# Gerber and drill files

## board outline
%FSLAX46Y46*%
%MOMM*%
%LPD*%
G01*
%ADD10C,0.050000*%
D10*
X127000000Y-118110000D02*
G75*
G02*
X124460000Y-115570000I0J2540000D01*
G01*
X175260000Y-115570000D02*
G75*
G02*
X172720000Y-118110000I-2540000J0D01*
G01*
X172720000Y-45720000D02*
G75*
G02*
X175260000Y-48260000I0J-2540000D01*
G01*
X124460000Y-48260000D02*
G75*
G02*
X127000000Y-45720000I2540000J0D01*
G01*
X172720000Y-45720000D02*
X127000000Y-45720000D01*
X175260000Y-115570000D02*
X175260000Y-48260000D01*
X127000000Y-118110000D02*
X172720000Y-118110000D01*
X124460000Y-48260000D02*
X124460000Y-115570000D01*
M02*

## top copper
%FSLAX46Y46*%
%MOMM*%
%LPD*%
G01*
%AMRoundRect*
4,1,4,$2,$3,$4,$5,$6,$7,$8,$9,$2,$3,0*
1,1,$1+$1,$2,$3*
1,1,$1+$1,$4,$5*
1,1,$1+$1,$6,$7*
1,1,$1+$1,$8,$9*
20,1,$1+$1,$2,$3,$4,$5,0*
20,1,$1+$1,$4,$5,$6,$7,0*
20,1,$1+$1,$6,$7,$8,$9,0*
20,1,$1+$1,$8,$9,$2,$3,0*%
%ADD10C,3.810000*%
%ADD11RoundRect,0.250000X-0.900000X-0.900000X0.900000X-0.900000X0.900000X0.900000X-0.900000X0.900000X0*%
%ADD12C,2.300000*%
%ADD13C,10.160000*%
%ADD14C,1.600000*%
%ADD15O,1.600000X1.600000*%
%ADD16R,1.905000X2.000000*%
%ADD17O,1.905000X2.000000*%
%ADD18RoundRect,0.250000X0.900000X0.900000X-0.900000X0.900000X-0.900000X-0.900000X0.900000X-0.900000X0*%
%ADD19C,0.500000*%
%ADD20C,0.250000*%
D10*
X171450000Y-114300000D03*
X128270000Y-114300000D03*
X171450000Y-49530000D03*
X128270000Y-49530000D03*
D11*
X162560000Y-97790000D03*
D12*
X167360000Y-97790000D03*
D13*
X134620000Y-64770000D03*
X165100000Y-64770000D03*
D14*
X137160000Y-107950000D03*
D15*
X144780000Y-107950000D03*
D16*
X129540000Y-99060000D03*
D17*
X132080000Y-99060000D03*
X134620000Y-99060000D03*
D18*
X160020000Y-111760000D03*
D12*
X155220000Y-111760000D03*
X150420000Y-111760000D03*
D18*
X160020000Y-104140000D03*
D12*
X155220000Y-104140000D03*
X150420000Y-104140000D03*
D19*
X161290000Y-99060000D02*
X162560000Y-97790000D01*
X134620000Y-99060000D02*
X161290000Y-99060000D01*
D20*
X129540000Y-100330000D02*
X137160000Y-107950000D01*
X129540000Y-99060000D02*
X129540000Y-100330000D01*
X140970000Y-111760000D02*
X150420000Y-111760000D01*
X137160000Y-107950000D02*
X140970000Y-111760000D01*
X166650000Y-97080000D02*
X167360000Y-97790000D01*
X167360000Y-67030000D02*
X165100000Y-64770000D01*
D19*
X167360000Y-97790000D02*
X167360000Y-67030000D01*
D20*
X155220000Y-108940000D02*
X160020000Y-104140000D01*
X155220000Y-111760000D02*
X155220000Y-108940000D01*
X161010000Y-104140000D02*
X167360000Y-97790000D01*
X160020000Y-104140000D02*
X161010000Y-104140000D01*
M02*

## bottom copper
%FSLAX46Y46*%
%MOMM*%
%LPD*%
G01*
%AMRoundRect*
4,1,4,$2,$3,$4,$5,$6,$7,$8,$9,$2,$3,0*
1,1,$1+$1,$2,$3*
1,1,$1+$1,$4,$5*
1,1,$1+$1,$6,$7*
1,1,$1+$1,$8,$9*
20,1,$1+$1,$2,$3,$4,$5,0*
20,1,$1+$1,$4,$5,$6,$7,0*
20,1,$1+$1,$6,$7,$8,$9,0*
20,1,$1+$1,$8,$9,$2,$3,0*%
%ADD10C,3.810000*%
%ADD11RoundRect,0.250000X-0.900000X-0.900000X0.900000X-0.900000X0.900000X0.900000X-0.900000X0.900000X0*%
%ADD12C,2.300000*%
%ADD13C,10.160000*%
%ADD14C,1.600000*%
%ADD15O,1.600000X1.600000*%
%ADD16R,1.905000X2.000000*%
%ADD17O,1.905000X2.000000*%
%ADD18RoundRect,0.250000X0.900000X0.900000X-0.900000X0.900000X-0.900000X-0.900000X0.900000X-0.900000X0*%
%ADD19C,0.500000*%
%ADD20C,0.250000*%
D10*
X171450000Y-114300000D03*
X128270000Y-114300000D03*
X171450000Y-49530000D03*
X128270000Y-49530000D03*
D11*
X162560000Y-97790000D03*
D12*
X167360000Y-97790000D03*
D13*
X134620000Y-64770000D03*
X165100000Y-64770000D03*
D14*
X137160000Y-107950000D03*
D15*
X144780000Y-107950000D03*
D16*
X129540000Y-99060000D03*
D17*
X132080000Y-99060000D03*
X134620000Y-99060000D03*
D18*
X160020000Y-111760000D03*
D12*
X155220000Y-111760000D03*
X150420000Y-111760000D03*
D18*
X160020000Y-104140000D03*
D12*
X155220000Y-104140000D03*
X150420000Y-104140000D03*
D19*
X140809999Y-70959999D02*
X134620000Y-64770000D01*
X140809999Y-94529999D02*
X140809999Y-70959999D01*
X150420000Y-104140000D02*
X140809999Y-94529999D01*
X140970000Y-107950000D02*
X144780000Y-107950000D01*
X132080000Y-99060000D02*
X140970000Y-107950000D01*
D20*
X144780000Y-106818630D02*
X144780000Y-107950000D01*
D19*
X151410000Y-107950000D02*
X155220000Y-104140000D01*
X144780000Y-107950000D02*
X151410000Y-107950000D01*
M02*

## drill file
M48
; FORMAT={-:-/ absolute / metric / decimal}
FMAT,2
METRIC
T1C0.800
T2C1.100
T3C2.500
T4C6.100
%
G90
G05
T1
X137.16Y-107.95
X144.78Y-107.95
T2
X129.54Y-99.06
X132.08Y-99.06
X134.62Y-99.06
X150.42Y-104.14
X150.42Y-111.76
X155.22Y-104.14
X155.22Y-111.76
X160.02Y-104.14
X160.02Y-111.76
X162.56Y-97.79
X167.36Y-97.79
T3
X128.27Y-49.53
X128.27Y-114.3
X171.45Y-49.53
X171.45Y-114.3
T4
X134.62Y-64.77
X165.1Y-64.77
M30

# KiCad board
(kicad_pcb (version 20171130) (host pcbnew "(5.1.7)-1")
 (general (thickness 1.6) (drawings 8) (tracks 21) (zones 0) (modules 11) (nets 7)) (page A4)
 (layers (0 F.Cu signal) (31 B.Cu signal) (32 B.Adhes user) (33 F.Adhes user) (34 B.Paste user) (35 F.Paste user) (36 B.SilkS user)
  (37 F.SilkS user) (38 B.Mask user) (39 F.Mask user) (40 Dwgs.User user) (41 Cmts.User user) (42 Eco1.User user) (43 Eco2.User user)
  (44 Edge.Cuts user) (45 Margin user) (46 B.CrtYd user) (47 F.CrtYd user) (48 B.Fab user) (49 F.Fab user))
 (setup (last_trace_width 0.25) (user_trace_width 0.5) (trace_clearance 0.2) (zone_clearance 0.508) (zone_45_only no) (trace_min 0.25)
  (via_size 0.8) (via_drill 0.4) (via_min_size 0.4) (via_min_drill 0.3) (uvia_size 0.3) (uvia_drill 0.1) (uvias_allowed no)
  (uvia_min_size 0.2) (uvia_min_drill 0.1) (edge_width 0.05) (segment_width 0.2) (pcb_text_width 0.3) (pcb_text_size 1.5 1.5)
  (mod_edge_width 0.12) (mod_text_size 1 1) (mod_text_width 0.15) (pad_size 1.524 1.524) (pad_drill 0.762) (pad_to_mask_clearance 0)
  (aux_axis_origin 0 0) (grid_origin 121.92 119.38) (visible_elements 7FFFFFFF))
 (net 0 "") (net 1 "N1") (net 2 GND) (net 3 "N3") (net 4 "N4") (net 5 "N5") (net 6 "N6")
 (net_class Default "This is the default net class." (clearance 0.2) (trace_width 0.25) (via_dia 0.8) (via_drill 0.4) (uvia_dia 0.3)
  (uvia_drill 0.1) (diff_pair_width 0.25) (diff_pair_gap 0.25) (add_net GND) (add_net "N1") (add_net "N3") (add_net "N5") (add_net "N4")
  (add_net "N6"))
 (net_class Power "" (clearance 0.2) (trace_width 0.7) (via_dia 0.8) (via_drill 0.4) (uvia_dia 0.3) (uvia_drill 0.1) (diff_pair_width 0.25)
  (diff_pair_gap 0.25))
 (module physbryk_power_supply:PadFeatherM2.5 (layer F.Cu) (at 171.45 114.3)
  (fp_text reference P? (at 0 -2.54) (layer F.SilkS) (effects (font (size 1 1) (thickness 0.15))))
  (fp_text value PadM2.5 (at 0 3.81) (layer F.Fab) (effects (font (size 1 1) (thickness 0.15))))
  (pad ? thru_hole circle (at 0 0) (size 3.81 3.81) (drill 2.5) (layers *.Cu *.Mask) (solder_mask_margin 0.0508)))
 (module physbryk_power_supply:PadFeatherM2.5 (layer F.Cu) (at 128.27 114.3)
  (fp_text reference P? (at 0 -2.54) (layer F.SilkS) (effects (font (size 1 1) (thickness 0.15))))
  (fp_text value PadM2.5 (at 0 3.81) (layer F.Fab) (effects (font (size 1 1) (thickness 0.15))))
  (pad ? thru_hole circle (at 0 0) (size 3.81 3.81) (drill 2.5) (layers *.Cu *.Mask) (solder_mask_margin 0.0508)))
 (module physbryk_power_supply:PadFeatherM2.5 (layer F.Cu) (at 171.45 49.53)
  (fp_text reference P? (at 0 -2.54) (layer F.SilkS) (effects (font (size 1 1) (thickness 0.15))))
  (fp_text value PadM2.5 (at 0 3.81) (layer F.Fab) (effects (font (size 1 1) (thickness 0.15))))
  (pad ? thru_hole circle (at 0 0) (size 3.81 3.81) (drill 2.5) (layers *.Cu *.Mask) (solder_mask_margin 0.0508)))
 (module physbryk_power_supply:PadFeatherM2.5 (layer F.Cu) (at 128.27 49.53)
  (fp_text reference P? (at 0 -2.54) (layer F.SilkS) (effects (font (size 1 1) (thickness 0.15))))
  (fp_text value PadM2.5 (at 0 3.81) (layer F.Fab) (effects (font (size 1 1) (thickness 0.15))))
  (pad ? thru_hole circle (at 0 0) (size 3.81 3.81) (drill 2.5) (layers *.Cu *.Mask) (solder_mask_margin 0.0508)))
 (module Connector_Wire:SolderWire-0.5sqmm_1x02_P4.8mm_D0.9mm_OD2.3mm (layer F.Cu) (at 162.56 97.79)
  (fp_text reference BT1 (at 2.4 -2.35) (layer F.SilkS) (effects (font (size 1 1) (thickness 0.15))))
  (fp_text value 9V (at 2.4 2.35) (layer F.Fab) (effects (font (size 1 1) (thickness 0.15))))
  (pad 1 thru_hole roundrect (at 0 0) (size 2.3 2.3) (drill 1.1) (layers *.Cu *.Mask) (roundrect_rratio 0.108695652173913) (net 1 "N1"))
  (pad 2 thru_hole circle (at 4.8 0) (size 2.3 2.3) (drill 1.1) (layers *.Cu *.Mask) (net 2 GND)))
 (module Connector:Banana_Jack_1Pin (layer F.Cu) (at 134.62 64.77)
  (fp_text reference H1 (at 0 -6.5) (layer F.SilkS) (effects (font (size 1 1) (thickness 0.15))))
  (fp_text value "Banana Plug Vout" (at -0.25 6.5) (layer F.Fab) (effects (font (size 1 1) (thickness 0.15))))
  (pad 1 thru_hole circle (at 0 0) (size 10.16 10.16) (drill 6.1) (layers *.Cu *.Mask) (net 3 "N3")))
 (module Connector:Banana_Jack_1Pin (layer F.Cu) (at 165.1 64.77)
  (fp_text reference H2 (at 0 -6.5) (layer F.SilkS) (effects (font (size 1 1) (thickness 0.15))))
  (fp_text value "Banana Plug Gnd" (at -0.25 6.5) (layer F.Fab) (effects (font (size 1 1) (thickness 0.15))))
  (pad 1 thru_hole circle (at 0 0) (size 10.16 10.16) (drill 6.1) (layers *.Cu *.Mask) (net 2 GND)))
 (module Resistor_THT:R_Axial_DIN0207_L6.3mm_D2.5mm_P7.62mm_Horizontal (layer F.Cu) (at 137.16 107.95)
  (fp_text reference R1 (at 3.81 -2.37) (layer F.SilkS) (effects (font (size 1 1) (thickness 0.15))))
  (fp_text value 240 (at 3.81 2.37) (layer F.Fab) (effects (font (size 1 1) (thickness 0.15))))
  (pad 1 thru_hole circle (at 0 0) (size 1.6 1.6) (drill 0.8) (layers *.Cu *.Mask) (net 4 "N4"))
  (pad 2 thru_hole oval (at 7.62 0) (size 1.6 1.6) (drill 0.8) (layers *.Cu *.Mask) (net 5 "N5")))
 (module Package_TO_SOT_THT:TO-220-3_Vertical (layer F.Cu) (at 129.54 99.06)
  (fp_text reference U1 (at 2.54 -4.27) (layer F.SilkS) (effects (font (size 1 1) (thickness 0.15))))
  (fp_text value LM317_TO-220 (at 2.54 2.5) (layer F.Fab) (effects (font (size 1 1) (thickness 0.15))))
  (pad 1 thru_hole rect (at 0 0) (size 1.905 2) (drill 1.1) (layers *.Cu *.Mask) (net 4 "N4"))
  (pad 2 thru_hole oval (at 2.54 0) (size 1.905 2) (drill 1.1) (layers *.Cu *.Mask) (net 5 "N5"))
  (pad 3 thru_hole oval (at 5.08 0) (size 1.905 2) (drill 1.1) (layers *.Cu *.Mask) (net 1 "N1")))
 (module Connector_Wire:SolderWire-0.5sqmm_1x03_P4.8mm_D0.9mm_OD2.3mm (layer F.Cu) (at 160.02 111.76 180)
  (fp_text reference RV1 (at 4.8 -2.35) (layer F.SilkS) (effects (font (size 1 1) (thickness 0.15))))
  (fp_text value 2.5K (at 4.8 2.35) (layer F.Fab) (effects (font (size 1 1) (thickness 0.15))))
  (pad 1 thru_hole roundrect (at 0 0 180) (size 2.3 2.3) (drill 1.1) (layers *.Cu *.Mask) (roundrect_rratio 0.108695652173913) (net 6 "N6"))
  (pad 2 thru_hole circle (at 4.8 0 180) (size 2.3 2.3) (drill 1.1) (layers *.Cu *.Mask) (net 2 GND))
  (pad 3 thru_hole circle (at 9.6 0 180) (size 2.3 2.3) (drill 1.1) (layers *.Cu *.Mask) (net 4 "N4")))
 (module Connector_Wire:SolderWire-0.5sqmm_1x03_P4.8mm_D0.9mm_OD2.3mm (layer F.Cu) (at 160.02 104.14 180)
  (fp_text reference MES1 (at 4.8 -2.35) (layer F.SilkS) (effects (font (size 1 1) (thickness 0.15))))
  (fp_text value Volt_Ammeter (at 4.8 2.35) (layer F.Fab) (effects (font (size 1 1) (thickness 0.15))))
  (pad 1 thru_hole roundrect (at 0 0 180) (size 2.3 2.3) (drill 1.1) (layers *.Cu *.Mask) (roundrect_rratio 0.108695652173913) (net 2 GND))
  (pad 2 thru_hole circle (at 4.8 0 180) (size 2.3 2.3) (drill 1.1) (layers *.Cu *.Mask) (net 5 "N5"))
  (pad 3 thru_hole circle (at 9.6 0 180) (size 2.3 2.3) (drill 1.1) (layers *.Cu *.Mask) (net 3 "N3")))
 (gr_arc (start 127 115.57) (end 124.46 115.57) (angle -90) (layer Edge.Cuts) (width 0.05))
 (gr_arc (start 172.72 115.57) (end 172.72 118.11) (angle -90) (layer Edge.Cuts) (width 0.05))
 (gr_arc (start 172.72 48.26) (end 175.26 48.26) (angle -90) (layer Edge.Cuts) (width 0.05))
 (gr_arc (start 127 48.26) (end 127 45.72) (angle -90) (layer Edge.Cuts) (width 0.05))
 (gr_line (start 172.72 45.72) (end 127 45.72) (layer Edge.Cuts) (width 0.05))
 (gr_line (start 175.26 115.57) (end 175.26 48.26) (layer Edge.Cuts) (width 0.05))
 (gr_line (start 127 118.11) (end 172.72 118.11) (layer Edge.Cuts) (width 0.05))
 (gr_line (start 124.46 48.26) (end 124.46 115.57) (layer Edge.Cuts) (width 0.05))
 (segment (start 161.29 99.06) (end 162.56 97.79) (width 0.5) (layer F.Cu) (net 1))
 (segment (start 134.62 99.06) (end 161.29 99.06) (width 0.5) (layer F.Cu) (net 1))
 (segment (start 140.809999 70.959999) (end 134.62 64.77) (width 0.5) (layer B.Cu) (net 3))
 (segment (start 140.809999 94.529999) (end 140.809999 70.959999) (width 0.5) (layer B.Cu) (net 3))
 (segment (start 150.42 104.14) (end 140.809999 94.529999) (width 0.5) (layer B.Cu) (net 3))
 (segment (start 129.54 100.33) (end 137.16 107.95) (width 0.25) (layer F.Cu) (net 4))
 (segment (start 129.54 99.06) (end 129.54 100.33) (width 0.25) (layer F.Cu) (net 4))
 (segment (start 140.97 111.76) (end 150.42 111.76) (width 0.25) (layer F.Cu) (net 4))
 (segment (start 137.16 107.95) (end 140.97 111.76) (width 0.25) (layer F.Cu) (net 4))
 (segment (start 166.65 97.08) (end 167.36 97.79) (width 0.25) (layer F.Cu) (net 2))
 (segment (start 167.36 67.03) (end 165.1 64.77) (width 0.25) (layer F.Cu) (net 2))
 (segment (start 167.36 97.79) (end 167.36 67.03) (width 0.5) (layer F.Cu) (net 2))
 (segment (start 155.22 108.94) (end 160.02 104.14) (width 0.25) (layer F.Cu) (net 2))
 (segment (start 155.22 111.76) (end 155.22 108.94) (width 0.25) (layer F.Cu) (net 2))
 (segment (start 161.01 104.14) (end 167.36 97.79) (width 0.25) (layer F.Cu) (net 2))
 (segment (start 160.02 104.14) (end 161.01 104.14) (width 0.25) (layer F.Cu) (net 2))
 (segment (start 140.97 107.95) (end 144.78 107.95) (width 0.5) (layer B.Cu) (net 5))
 (segment (start 132.08 99.06) (end 140.97 107.95) (width 0.5) (layer B.Cu) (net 5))
 (segment (start 144.78 106.81863) (end 144.78 107.95) (width 0.25) (layer B.Cu) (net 5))
 (segment (start 151.41 107.95) (end 155.22 104.14) (width 0.5) (layer B.Cu) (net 5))
 (segment (start 144.78 107.95) (end 151.41 107.95) (width 0.5) (layer B.Cu) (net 5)))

